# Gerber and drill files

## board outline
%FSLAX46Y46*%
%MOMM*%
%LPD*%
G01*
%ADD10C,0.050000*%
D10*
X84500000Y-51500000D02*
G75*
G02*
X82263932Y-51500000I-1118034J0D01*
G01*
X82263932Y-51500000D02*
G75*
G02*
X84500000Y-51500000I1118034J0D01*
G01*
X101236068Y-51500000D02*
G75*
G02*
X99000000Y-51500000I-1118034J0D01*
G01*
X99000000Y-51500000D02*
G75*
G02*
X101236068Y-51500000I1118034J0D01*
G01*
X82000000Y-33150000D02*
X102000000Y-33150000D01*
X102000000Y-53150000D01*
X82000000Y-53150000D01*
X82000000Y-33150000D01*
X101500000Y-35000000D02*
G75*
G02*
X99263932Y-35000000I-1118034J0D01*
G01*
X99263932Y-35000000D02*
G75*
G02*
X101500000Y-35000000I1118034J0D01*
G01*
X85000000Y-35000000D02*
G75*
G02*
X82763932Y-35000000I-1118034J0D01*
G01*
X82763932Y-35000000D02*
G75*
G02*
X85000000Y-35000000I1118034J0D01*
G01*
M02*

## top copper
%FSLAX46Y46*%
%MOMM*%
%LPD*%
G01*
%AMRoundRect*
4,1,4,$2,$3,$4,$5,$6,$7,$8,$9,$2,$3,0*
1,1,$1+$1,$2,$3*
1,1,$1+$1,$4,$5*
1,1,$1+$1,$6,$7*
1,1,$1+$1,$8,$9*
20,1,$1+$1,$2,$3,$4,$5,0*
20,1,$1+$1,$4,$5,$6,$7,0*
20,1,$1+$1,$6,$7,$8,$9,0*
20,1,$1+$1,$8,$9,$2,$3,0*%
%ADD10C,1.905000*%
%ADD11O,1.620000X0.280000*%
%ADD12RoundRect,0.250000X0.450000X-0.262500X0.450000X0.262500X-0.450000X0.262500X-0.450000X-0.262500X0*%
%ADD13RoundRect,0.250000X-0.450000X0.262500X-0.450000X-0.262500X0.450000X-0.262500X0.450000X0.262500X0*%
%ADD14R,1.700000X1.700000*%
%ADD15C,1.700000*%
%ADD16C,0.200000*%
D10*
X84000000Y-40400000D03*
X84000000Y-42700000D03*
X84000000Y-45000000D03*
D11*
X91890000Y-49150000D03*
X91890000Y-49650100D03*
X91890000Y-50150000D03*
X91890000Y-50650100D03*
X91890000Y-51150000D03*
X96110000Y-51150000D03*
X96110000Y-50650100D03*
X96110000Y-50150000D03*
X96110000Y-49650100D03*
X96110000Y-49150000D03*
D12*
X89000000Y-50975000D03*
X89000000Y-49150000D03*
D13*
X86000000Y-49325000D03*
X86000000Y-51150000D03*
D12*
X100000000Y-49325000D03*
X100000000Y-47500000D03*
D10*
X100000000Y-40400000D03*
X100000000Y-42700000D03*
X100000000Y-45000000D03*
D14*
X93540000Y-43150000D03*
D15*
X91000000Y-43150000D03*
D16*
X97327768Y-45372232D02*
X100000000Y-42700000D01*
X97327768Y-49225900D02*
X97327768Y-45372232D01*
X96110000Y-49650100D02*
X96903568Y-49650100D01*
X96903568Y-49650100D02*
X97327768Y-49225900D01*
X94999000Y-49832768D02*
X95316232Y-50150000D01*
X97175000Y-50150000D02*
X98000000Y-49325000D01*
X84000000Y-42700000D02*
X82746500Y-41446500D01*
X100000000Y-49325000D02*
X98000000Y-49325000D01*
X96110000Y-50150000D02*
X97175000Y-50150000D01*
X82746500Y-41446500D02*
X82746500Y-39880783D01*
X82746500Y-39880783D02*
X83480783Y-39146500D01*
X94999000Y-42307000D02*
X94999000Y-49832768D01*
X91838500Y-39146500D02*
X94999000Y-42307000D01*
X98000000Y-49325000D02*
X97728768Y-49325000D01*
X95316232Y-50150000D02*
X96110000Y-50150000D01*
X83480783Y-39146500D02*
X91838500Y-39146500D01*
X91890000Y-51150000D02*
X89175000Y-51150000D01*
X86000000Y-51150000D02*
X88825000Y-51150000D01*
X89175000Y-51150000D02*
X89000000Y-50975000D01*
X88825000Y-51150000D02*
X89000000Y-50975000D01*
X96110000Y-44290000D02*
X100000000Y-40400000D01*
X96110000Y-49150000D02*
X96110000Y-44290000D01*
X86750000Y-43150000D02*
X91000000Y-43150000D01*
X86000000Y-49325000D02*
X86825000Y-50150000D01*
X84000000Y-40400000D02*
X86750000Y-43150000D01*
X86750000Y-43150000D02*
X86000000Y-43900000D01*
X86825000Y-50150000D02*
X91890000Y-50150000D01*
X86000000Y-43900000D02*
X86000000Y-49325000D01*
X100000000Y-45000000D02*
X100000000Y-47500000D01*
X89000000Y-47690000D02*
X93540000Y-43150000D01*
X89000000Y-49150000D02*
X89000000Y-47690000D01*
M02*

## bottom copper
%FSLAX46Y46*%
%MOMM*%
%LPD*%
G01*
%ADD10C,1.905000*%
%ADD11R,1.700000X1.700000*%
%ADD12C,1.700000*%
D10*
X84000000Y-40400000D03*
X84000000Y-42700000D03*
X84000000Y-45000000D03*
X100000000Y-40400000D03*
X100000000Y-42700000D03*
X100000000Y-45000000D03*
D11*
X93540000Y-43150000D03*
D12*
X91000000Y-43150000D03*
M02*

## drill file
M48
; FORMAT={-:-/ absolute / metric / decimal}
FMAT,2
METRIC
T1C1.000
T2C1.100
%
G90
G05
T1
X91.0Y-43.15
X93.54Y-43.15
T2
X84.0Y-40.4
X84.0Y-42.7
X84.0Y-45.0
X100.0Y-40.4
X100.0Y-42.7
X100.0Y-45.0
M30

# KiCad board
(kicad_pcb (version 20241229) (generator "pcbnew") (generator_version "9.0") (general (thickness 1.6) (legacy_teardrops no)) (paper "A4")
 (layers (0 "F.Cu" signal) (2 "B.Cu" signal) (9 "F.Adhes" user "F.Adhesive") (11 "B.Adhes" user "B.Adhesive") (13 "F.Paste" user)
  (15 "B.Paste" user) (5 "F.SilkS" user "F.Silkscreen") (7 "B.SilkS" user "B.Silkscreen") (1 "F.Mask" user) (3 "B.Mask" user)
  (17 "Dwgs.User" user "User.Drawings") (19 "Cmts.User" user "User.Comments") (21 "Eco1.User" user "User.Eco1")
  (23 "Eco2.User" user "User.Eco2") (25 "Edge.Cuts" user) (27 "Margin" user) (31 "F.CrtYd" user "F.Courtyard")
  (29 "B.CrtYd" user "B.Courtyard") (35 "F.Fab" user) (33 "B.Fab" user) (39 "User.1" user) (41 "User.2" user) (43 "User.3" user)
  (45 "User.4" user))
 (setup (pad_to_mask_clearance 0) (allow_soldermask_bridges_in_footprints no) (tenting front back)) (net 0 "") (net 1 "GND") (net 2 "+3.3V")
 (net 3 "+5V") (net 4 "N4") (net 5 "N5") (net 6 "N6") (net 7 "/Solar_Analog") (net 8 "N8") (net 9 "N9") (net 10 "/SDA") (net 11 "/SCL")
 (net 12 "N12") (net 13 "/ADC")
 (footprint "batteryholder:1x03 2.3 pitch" (layer "F.Cu") (at 84 40.4 -90)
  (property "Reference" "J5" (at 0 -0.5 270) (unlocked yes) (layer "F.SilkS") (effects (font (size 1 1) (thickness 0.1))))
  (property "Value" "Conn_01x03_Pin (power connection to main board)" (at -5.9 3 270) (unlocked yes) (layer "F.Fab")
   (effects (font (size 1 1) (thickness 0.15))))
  (pad "1" thru_hole circle (at 0 0 270) (size 1.905 1.905) (drill 1.1) (layers "*.Cu" "*.Mask") (remove_unused_layers no) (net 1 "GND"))
  (pad "2" thru_hole circle (at 2.3 0 270) (size 1.905 1.905) (drill 1.1) (layers "*.Cu" "*.Mask") (remove_unused_layers no) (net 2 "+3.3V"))
  (pad "3" thru_hole circle (at 4.6 0 270) (size 1.905 1.905) (drill 1.1) (layers "*.Cu" "*.Mask") (remove_unused_layers no) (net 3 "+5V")))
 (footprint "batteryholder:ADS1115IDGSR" (layer "F.Cu") (at 94 50.15 -90)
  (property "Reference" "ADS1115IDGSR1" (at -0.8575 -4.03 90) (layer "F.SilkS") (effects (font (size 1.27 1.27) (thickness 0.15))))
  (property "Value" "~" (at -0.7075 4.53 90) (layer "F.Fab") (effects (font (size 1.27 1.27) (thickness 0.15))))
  (pad "1" smd oval (at -1 2.11 270) (size 0.28 1.62) (layers "F.Cu" "F.Mask" "F.Paste") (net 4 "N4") (solder_mask_margin 0.0508)
   (solder_paste_margin 0) (thermal_bridge_angle 0))
  (pad "2" smd oval (at -0.4999 2.11 270) (size 0.28 1.62) (layers "F.Cu" "F.Mask" "F.Paste") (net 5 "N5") (solder_mask_margin 0.0508)
   (solder_paste_margin 0) (thermal_bridge_angle 0))
  (pad "3" smd oval (at 0 2.11 270) (size 0.28 1.62) (layers "F.Cu" "F.Mask" "F.Paste") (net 1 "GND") (solder_mask_margin 0.0508)
   (solder_paste_margin 0) (thermal_bridge_angle 0))
  (pad "4" smd oval (at 0.5001 2.11 270) (size 0.28 1.62) (layers "F.Cu" "F.Mask" "F.Paste") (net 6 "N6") (solder_mask_margin 0.0508)
   (solder_paste_margin 0) (thermal_bridge_angle 0))
  (pad "5" smd oval (at 1 2.11 270) (size 0.28 1.62) (layers "F.Cu" "F.Mask" "F.Paste") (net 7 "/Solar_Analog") (solder_mask_margin 0.0508)
   (solder_paste_margin 0) (thermal_bridge_angle 0))
  (pad "6" smd oval (at 1 -2.11 270) (size 0.28 1.62) (layers "F.Cu" "F.Mask" "F.Paste") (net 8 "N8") (solder_mask_margin 0.0508)
   (solder_paste_margin 0) (thermal_bridge_angle 0))
  (pad "7" smd oval (at 0.5001 -2.11 270) (size 0.28 1.62) (layers "F.Cu" "F.Mask" "F.Paste") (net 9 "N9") (solder_mask_margin 0.0508)
   (solder_paste_margin 0) (thermal_bridge_angle 0))
  (pad "8" smd oval (at 0 -2.11 270) (size 0.28 1.62) (layers "F.Cu" "F.Mask" "F.Paste") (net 2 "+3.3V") (solder_mask_margin 0.0508)
   (solder_paste_margin 0) (thermal_bridge_angle 0))
  (pad "9" smd oval (at -0.4999 -2.11 270) (size 0.28 1.62) (layers "F.Cu" "F.Mask" "F.Paste") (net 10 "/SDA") (solder_mask_margin 0.0508)
   (solder_paste_margin 0) (thermal_bridge_angle 0))
  (pad "10" smd oval (at -1 -2.11 270) (size 0.28 1.62) (layers "F.Cu" "F.Mask" "F.Paste") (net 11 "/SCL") (solder_mask_margin 0.0508)
   (solder_paste_margin 0) (thermal_bridge_angle 0))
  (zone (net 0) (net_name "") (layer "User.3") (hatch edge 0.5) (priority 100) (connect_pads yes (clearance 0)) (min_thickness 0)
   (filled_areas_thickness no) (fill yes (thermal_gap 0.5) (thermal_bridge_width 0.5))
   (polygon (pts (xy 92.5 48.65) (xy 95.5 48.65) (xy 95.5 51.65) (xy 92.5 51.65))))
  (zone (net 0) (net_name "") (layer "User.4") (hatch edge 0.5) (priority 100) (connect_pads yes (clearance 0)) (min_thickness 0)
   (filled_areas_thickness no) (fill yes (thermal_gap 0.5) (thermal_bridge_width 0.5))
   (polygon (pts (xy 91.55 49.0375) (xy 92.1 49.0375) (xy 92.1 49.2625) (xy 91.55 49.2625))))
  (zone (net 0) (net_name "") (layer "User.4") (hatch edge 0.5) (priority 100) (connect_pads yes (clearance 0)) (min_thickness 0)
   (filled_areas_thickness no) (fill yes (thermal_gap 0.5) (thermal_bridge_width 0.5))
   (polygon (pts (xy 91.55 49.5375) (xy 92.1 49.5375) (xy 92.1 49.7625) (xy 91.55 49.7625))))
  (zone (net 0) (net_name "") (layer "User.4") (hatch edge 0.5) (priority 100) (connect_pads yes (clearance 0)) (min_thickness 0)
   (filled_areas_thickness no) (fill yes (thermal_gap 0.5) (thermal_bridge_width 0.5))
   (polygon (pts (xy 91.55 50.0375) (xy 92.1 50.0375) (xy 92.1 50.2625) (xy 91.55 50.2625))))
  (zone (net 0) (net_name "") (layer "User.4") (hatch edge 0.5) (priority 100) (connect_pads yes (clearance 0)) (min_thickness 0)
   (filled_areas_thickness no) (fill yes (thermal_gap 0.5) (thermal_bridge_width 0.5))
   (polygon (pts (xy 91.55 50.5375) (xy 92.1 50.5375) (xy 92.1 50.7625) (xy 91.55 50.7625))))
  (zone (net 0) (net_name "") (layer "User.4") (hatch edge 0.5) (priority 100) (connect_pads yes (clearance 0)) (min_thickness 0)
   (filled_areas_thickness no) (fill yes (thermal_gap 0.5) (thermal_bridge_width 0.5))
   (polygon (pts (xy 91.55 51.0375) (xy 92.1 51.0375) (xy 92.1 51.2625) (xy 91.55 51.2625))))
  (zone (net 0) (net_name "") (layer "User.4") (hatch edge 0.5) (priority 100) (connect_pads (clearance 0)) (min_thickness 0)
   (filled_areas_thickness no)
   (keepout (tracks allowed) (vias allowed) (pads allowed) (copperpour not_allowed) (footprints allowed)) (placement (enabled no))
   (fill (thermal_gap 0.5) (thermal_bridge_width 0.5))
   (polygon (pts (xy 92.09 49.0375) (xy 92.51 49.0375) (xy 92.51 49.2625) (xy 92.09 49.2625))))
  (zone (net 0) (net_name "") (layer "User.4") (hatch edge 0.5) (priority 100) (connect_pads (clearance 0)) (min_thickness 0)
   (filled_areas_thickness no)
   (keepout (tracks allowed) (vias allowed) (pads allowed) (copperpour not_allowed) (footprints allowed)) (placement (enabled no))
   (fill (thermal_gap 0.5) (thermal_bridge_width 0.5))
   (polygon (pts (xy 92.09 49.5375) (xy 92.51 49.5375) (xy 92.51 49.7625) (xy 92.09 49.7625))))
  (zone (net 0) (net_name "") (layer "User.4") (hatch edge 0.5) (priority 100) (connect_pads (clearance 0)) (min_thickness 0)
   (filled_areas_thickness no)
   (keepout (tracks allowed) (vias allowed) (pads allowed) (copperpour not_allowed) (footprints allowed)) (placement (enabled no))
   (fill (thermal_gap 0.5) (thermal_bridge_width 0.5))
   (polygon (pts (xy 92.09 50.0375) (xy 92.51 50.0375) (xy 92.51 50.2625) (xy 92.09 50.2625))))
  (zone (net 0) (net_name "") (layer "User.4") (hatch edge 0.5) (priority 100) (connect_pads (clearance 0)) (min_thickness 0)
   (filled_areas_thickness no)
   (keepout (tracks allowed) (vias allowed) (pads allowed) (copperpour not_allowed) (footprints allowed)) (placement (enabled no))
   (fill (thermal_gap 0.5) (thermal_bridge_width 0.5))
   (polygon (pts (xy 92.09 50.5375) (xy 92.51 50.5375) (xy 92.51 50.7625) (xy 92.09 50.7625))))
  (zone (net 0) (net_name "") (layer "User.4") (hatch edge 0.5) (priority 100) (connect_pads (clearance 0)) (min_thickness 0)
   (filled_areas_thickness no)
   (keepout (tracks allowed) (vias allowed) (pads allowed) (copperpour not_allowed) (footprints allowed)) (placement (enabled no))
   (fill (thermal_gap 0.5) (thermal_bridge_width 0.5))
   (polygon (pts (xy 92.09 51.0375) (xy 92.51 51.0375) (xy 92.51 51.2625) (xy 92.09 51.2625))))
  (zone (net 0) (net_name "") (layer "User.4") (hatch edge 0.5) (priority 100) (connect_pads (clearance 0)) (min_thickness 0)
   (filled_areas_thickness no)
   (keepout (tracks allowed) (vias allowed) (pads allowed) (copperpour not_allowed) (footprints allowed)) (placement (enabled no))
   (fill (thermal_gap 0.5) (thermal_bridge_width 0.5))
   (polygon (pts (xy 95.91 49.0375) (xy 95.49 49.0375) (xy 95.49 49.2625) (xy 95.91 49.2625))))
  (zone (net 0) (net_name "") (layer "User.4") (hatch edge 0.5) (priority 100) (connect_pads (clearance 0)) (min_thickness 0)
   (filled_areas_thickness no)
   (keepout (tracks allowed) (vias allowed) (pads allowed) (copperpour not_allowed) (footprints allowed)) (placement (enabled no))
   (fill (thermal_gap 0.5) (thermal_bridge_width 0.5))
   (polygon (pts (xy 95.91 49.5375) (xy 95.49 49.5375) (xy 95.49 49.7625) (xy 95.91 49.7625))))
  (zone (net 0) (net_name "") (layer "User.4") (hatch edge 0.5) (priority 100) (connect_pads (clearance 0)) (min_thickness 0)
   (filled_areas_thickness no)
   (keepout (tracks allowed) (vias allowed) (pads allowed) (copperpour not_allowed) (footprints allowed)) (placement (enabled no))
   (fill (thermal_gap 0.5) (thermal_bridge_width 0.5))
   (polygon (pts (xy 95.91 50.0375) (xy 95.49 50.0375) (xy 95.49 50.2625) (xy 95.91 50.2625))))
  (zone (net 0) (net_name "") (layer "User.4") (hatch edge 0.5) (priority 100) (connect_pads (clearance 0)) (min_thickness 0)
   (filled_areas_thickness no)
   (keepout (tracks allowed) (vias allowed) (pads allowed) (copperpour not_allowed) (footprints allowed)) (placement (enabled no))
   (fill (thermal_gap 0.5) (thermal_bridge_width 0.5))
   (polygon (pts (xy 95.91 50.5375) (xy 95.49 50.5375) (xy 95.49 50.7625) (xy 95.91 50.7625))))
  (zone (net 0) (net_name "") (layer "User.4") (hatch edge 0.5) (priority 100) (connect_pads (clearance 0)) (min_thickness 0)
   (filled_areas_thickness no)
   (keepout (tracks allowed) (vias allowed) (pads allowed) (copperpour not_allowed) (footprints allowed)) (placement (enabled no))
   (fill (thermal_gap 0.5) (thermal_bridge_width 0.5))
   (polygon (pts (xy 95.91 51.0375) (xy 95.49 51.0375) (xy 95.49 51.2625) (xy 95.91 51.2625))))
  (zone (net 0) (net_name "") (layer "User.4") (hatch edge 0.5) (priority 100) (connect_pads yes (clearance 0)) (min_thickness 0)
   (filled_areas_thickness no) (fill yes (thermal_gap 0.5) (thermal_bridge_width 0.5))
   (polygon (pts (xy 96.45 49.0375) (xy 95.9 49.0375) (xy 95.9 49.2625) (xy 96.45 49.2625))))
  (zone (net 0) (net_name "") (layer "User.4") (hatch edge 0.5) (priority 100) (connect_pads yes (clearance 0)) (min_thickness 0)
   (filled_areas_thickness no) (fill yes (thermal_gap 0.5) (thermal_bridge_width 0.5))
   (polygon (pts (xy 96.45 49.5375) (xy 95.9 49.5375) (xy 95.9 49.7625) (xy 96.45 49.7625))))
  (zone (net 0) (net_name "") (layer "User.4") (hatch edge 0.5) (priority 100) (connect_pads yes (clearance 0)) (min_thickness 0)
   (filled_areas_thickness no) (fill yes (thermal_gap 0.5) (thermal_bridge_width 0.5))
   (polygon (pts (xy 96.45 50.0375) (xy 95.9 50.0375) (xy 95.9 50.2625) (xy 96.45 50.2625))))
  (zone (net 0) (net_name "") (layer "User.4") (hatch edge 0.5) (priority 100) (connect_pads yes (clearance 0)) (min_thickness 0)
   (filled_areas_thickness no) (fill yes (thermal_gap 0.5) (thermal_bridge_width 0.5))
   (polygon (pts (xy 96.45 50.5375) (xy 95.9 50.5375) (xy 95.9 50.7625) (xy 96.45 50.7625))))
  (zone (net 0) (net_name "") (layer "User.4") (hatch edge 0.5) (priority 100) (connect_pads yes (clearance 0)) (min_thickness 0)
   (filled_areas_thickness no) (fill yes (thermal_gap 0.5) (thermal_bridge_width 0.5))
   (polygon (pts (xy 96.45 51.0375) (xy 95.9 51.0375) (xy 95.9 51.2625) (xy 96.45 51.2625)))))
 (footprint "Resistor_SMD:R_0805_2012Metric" (layer "F.Cu") (at 89 50.0625 90)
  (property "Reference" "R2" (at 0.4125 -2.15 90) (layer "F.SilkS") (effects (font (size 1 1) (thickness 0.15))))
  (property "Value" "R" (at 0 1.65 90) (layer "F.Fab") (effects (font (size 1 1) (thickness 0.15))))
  (pad "1" smd roundrect (at -0.9125 0 90) (size 1.025 1.4) (layers "F.Cu" "F.Mask" "F.Paste") (roundrect_rratio 0.243902)
   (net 7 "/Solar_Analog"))
  (pad "2" smd roundrect (at 0.9125 0 90) (size 1.025 1.4) (layers "F.Cu" "F.Mask" "F.Paste") (roundrect_rratio 0.243902) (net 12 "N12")))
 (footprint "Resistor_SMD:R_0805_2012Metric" (layer "F.Cu") (at 86 50.2375 -90)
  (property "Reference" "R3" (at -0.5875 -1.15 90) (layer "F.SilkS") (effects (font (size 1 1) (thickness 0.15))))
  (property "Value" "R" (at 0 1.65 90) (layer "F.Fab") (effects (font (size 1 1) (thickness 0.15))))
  (pad "1" smd roundrect (at -0.9125 0 270) (size 1.025 1.4) (layers "F.Cu" "F.Mask" "F.Paste") (roundrect_rratio 0.243902) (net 1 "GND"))
  (pad "2" smd roundrect (at 0.9125 0 270) (size 1.025 1.4) (layers "F.Cu" "F.Mask" "F.Paste") (roundrect_rratio 0.243902)
   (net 7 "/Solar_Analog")))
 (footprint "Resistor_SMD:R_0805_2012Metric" (layer "F.Cu") (at 100 48.4125 90)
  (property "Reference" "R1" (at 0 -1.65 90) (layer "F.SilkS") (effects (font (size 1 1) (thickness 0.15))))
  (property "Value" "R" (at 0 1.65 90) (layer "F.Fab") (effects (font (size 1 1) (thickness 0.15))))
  (pad "1" smd roundrect (at -0.9125 0 90) (size 1.025 1.4) (layers "F.Cu" "F.Mask" "F.Paste") (roundrect_rratio 0.243902) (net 2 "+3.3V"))
  (pad "2" smd roundrect (at 0.9125 0 90) (size 1.025 1.4) (layers "F.Cu" "F.Mask" "F.Paste") (roundrect_rratio 0.243902) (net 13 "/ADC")))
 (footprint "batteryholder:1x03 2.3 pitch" (layer "F.Cu") (at 100 40.4 -90)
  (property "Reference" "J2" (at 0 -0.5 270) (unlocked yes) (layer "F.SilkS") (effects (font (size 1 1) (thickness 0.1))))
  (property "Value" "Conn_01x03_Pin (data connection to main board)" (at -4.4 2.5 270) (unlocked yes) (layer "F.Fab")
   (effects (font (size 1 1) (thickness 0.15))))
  (pad "1" thru_hole circle (at 0 0 270) (size 1.905 1.905) (drill 1.1) (layers "*.Cu" "*.Mask") (remove_unused_layers no) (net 11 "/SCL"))
  (pad "2" thru_hole circle (at 2.3 0 270) (size 1.905 1.905) (drill 1.1) (layers "*.Cu" "*.Mask") (remove_unused_layers no) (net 10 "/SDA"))
  (pad "3" thru_hole circle (at 4.6 0 270) (size 1.905 1.905) (drill 1.1) (layers "*.Cu" "*.Mask") (remove_unused_layers no) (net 13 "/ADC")))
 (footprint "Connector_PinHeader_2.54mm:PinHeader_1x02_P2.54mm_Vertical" (layer "F.Cu") (at 93.54 43.15 -90)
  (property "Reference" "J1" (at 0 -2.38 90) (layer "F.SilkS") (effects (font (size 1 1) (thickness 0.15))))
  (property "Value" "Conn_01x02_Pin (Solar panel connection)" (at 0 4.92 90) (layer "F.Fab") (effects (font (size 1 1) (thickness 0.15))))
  (pad "1" thru_hole rect (at 0 0 270) (size 1.7 1.7) (drill 1) (layers "*.Cu" "*.Mask") (remove_unused_layers no) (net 12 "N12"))
  (pad "2" thru_hole circle (at 0 2.54 270) (size 1.7 1.7) (drill 1) (layers "*.Cu" "*.Mask") (remove_unused_layers no) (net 1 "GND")))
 (gr_circle (center 83.381966 51.5) (end 84.381966 52) (stroke (width 0.05) (type default)) (fill no) (layer "Edge.Cuts"))
 (gr_circle (center 100.118034 51.5) (end 101.118034 52) (stroke (width 0.05) (type default)) (fill no) (layer "Edge.Cuts"))
 (gr_rect (start 82 33.15) (end 102 53.15) (stroke (width 0.05) (type default)) (fill no) (layer "Edge.Cuts"))
 (gr_circle (center 100.381966 35) (end 101.381966 35.5) (stroke (width 0.05) (type default)) (fill no) (layer "Edge.Cuts"))
 (gr_circle (center 83.881966 35) (end 84.881966 35.5) (stroke (width 0.05) (type default)) (fill no) (layer "Edge.Cuts"))
 (segment (start 97.327768 45.372232) (end 100 42.7) (width 0.2) (layer "F.Cu") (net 10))
 (segment (start 97.327768 49.2259) (end 97.327768 45.372232) (width 0.2) (layer "F.Cu") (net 10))
 (segment (start 96.11 49.6501) (end 96.903568 49.6501) (width 0.2) (layer "F.Cu") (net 10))
 (segment (start 96.903568 49.6501) (end 97.327768 49.2259) (width 0.2) (layer "F.Cu") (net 10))
 (segment (start 94.999 49.832768) (end 95.316232 50.15) (width 0.2) (layer "F.Cu") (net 2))
 (segment (start 97.175 50.15) (end 98 49.325) (width 0.2) (layer "F.Cu") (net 2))
 (segment (start 84 42.7) (end 82.7465 41.4465) (width 0.2) (layer "F.Cu") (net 2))
 (segment (start 100 49.325) (end 98 49.325) (width 0.2) (layer "F.Cu") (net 2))
 (segment (start 96.11 50.15) (end 97.175 50.15) (width 0.2) (layer "F.Cu") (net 2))
 (segment (start 82.7465 41.4465) (end 82.7465 39.880783) (width 0.2) (layer "F.Cu") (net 2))
 (segment (start 82.7465 39.880783) (end 83.480783 39.1465) (width 0.2) (layer "F.Cu") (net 2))
 (segment (start 94.999 42.307) (end 94.999 49.832768) (width 0.2) (layer "F.Cu") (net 2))
 (segment (start 91.8385 39.1465) (end 94.999 42.307) (width 0.2) (layer "F.Cu") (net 2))
 (segment (start 98 49.325) (end 97.728768 49.325) (width 0.2) (layer "F.Cu") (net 2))
 (segment (start 95.316232 50.15) (end 96.11 50.15) (width 0.2) (layer "F.Cu") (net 2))
 (segment (start 83.480783 39.1465) (end 91.8385 39.1465) (width 0.2) (layer "F.Cu") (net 2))
 (segment (start 91.89 51.15) (end 89.175 51.15) (width 0.2) (layer "F.Cu") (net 7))
 (segment (start 86 51.15) (end 88.825 51.15) (width 0.2) (layer "F.Cu") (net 7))
 (segment (start 89.175 51.15) (end 89 50.975) (width 0.2) (layer "F.Cu") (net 7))
 (segment (start 88.825 51.15) (end 89 50.975) (width 0.2) (layer "F.Cu") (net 7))
 (segment (start 96.11 44.29) (end 100 40.4) (width 0.2) (layer "F.Cu") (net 11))
 (segment (start 96.11 49.15) (end 96.11 44.29) (width 0.2) (layer "F.Cu") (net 11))
 (segment (start 86.75 43.15) (end 91 43.15) (width 0.2) (layer "F.Cu") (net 1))
 (segment (start 86 49.325) (end 86.825 50.15) (width 0.2) (layer "F.Cu") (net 1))
 (segment (start 84 40.4) (end 86.75 43.15) (width 0.2) (layer "F.Cu") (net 1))
 (segment (start 86.75 43.15) (end 86 43.9) (width 0.2) (layer "F.Cu") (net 1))
 (segment (start 86.825 50.15) (end 91.89 50.15) (width 0.2) (layer "F.Cu") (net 1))
 (segment (start 86 43.9) (end 86 49.325) (width 0.2) (layer "F.Cu") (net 1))
 (segment (start 100 45) (end 100 47.5) (width 0.2) (layer "F.Cu") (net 13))
 (segment (start 89 47.69) (end 93.54 43.15) (width 0.2) (layer "F.Cu") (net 12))
 (segment (start 89 49.15) (end 89 47.69) (width 0.2) (layer "F.Cu") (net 12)))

